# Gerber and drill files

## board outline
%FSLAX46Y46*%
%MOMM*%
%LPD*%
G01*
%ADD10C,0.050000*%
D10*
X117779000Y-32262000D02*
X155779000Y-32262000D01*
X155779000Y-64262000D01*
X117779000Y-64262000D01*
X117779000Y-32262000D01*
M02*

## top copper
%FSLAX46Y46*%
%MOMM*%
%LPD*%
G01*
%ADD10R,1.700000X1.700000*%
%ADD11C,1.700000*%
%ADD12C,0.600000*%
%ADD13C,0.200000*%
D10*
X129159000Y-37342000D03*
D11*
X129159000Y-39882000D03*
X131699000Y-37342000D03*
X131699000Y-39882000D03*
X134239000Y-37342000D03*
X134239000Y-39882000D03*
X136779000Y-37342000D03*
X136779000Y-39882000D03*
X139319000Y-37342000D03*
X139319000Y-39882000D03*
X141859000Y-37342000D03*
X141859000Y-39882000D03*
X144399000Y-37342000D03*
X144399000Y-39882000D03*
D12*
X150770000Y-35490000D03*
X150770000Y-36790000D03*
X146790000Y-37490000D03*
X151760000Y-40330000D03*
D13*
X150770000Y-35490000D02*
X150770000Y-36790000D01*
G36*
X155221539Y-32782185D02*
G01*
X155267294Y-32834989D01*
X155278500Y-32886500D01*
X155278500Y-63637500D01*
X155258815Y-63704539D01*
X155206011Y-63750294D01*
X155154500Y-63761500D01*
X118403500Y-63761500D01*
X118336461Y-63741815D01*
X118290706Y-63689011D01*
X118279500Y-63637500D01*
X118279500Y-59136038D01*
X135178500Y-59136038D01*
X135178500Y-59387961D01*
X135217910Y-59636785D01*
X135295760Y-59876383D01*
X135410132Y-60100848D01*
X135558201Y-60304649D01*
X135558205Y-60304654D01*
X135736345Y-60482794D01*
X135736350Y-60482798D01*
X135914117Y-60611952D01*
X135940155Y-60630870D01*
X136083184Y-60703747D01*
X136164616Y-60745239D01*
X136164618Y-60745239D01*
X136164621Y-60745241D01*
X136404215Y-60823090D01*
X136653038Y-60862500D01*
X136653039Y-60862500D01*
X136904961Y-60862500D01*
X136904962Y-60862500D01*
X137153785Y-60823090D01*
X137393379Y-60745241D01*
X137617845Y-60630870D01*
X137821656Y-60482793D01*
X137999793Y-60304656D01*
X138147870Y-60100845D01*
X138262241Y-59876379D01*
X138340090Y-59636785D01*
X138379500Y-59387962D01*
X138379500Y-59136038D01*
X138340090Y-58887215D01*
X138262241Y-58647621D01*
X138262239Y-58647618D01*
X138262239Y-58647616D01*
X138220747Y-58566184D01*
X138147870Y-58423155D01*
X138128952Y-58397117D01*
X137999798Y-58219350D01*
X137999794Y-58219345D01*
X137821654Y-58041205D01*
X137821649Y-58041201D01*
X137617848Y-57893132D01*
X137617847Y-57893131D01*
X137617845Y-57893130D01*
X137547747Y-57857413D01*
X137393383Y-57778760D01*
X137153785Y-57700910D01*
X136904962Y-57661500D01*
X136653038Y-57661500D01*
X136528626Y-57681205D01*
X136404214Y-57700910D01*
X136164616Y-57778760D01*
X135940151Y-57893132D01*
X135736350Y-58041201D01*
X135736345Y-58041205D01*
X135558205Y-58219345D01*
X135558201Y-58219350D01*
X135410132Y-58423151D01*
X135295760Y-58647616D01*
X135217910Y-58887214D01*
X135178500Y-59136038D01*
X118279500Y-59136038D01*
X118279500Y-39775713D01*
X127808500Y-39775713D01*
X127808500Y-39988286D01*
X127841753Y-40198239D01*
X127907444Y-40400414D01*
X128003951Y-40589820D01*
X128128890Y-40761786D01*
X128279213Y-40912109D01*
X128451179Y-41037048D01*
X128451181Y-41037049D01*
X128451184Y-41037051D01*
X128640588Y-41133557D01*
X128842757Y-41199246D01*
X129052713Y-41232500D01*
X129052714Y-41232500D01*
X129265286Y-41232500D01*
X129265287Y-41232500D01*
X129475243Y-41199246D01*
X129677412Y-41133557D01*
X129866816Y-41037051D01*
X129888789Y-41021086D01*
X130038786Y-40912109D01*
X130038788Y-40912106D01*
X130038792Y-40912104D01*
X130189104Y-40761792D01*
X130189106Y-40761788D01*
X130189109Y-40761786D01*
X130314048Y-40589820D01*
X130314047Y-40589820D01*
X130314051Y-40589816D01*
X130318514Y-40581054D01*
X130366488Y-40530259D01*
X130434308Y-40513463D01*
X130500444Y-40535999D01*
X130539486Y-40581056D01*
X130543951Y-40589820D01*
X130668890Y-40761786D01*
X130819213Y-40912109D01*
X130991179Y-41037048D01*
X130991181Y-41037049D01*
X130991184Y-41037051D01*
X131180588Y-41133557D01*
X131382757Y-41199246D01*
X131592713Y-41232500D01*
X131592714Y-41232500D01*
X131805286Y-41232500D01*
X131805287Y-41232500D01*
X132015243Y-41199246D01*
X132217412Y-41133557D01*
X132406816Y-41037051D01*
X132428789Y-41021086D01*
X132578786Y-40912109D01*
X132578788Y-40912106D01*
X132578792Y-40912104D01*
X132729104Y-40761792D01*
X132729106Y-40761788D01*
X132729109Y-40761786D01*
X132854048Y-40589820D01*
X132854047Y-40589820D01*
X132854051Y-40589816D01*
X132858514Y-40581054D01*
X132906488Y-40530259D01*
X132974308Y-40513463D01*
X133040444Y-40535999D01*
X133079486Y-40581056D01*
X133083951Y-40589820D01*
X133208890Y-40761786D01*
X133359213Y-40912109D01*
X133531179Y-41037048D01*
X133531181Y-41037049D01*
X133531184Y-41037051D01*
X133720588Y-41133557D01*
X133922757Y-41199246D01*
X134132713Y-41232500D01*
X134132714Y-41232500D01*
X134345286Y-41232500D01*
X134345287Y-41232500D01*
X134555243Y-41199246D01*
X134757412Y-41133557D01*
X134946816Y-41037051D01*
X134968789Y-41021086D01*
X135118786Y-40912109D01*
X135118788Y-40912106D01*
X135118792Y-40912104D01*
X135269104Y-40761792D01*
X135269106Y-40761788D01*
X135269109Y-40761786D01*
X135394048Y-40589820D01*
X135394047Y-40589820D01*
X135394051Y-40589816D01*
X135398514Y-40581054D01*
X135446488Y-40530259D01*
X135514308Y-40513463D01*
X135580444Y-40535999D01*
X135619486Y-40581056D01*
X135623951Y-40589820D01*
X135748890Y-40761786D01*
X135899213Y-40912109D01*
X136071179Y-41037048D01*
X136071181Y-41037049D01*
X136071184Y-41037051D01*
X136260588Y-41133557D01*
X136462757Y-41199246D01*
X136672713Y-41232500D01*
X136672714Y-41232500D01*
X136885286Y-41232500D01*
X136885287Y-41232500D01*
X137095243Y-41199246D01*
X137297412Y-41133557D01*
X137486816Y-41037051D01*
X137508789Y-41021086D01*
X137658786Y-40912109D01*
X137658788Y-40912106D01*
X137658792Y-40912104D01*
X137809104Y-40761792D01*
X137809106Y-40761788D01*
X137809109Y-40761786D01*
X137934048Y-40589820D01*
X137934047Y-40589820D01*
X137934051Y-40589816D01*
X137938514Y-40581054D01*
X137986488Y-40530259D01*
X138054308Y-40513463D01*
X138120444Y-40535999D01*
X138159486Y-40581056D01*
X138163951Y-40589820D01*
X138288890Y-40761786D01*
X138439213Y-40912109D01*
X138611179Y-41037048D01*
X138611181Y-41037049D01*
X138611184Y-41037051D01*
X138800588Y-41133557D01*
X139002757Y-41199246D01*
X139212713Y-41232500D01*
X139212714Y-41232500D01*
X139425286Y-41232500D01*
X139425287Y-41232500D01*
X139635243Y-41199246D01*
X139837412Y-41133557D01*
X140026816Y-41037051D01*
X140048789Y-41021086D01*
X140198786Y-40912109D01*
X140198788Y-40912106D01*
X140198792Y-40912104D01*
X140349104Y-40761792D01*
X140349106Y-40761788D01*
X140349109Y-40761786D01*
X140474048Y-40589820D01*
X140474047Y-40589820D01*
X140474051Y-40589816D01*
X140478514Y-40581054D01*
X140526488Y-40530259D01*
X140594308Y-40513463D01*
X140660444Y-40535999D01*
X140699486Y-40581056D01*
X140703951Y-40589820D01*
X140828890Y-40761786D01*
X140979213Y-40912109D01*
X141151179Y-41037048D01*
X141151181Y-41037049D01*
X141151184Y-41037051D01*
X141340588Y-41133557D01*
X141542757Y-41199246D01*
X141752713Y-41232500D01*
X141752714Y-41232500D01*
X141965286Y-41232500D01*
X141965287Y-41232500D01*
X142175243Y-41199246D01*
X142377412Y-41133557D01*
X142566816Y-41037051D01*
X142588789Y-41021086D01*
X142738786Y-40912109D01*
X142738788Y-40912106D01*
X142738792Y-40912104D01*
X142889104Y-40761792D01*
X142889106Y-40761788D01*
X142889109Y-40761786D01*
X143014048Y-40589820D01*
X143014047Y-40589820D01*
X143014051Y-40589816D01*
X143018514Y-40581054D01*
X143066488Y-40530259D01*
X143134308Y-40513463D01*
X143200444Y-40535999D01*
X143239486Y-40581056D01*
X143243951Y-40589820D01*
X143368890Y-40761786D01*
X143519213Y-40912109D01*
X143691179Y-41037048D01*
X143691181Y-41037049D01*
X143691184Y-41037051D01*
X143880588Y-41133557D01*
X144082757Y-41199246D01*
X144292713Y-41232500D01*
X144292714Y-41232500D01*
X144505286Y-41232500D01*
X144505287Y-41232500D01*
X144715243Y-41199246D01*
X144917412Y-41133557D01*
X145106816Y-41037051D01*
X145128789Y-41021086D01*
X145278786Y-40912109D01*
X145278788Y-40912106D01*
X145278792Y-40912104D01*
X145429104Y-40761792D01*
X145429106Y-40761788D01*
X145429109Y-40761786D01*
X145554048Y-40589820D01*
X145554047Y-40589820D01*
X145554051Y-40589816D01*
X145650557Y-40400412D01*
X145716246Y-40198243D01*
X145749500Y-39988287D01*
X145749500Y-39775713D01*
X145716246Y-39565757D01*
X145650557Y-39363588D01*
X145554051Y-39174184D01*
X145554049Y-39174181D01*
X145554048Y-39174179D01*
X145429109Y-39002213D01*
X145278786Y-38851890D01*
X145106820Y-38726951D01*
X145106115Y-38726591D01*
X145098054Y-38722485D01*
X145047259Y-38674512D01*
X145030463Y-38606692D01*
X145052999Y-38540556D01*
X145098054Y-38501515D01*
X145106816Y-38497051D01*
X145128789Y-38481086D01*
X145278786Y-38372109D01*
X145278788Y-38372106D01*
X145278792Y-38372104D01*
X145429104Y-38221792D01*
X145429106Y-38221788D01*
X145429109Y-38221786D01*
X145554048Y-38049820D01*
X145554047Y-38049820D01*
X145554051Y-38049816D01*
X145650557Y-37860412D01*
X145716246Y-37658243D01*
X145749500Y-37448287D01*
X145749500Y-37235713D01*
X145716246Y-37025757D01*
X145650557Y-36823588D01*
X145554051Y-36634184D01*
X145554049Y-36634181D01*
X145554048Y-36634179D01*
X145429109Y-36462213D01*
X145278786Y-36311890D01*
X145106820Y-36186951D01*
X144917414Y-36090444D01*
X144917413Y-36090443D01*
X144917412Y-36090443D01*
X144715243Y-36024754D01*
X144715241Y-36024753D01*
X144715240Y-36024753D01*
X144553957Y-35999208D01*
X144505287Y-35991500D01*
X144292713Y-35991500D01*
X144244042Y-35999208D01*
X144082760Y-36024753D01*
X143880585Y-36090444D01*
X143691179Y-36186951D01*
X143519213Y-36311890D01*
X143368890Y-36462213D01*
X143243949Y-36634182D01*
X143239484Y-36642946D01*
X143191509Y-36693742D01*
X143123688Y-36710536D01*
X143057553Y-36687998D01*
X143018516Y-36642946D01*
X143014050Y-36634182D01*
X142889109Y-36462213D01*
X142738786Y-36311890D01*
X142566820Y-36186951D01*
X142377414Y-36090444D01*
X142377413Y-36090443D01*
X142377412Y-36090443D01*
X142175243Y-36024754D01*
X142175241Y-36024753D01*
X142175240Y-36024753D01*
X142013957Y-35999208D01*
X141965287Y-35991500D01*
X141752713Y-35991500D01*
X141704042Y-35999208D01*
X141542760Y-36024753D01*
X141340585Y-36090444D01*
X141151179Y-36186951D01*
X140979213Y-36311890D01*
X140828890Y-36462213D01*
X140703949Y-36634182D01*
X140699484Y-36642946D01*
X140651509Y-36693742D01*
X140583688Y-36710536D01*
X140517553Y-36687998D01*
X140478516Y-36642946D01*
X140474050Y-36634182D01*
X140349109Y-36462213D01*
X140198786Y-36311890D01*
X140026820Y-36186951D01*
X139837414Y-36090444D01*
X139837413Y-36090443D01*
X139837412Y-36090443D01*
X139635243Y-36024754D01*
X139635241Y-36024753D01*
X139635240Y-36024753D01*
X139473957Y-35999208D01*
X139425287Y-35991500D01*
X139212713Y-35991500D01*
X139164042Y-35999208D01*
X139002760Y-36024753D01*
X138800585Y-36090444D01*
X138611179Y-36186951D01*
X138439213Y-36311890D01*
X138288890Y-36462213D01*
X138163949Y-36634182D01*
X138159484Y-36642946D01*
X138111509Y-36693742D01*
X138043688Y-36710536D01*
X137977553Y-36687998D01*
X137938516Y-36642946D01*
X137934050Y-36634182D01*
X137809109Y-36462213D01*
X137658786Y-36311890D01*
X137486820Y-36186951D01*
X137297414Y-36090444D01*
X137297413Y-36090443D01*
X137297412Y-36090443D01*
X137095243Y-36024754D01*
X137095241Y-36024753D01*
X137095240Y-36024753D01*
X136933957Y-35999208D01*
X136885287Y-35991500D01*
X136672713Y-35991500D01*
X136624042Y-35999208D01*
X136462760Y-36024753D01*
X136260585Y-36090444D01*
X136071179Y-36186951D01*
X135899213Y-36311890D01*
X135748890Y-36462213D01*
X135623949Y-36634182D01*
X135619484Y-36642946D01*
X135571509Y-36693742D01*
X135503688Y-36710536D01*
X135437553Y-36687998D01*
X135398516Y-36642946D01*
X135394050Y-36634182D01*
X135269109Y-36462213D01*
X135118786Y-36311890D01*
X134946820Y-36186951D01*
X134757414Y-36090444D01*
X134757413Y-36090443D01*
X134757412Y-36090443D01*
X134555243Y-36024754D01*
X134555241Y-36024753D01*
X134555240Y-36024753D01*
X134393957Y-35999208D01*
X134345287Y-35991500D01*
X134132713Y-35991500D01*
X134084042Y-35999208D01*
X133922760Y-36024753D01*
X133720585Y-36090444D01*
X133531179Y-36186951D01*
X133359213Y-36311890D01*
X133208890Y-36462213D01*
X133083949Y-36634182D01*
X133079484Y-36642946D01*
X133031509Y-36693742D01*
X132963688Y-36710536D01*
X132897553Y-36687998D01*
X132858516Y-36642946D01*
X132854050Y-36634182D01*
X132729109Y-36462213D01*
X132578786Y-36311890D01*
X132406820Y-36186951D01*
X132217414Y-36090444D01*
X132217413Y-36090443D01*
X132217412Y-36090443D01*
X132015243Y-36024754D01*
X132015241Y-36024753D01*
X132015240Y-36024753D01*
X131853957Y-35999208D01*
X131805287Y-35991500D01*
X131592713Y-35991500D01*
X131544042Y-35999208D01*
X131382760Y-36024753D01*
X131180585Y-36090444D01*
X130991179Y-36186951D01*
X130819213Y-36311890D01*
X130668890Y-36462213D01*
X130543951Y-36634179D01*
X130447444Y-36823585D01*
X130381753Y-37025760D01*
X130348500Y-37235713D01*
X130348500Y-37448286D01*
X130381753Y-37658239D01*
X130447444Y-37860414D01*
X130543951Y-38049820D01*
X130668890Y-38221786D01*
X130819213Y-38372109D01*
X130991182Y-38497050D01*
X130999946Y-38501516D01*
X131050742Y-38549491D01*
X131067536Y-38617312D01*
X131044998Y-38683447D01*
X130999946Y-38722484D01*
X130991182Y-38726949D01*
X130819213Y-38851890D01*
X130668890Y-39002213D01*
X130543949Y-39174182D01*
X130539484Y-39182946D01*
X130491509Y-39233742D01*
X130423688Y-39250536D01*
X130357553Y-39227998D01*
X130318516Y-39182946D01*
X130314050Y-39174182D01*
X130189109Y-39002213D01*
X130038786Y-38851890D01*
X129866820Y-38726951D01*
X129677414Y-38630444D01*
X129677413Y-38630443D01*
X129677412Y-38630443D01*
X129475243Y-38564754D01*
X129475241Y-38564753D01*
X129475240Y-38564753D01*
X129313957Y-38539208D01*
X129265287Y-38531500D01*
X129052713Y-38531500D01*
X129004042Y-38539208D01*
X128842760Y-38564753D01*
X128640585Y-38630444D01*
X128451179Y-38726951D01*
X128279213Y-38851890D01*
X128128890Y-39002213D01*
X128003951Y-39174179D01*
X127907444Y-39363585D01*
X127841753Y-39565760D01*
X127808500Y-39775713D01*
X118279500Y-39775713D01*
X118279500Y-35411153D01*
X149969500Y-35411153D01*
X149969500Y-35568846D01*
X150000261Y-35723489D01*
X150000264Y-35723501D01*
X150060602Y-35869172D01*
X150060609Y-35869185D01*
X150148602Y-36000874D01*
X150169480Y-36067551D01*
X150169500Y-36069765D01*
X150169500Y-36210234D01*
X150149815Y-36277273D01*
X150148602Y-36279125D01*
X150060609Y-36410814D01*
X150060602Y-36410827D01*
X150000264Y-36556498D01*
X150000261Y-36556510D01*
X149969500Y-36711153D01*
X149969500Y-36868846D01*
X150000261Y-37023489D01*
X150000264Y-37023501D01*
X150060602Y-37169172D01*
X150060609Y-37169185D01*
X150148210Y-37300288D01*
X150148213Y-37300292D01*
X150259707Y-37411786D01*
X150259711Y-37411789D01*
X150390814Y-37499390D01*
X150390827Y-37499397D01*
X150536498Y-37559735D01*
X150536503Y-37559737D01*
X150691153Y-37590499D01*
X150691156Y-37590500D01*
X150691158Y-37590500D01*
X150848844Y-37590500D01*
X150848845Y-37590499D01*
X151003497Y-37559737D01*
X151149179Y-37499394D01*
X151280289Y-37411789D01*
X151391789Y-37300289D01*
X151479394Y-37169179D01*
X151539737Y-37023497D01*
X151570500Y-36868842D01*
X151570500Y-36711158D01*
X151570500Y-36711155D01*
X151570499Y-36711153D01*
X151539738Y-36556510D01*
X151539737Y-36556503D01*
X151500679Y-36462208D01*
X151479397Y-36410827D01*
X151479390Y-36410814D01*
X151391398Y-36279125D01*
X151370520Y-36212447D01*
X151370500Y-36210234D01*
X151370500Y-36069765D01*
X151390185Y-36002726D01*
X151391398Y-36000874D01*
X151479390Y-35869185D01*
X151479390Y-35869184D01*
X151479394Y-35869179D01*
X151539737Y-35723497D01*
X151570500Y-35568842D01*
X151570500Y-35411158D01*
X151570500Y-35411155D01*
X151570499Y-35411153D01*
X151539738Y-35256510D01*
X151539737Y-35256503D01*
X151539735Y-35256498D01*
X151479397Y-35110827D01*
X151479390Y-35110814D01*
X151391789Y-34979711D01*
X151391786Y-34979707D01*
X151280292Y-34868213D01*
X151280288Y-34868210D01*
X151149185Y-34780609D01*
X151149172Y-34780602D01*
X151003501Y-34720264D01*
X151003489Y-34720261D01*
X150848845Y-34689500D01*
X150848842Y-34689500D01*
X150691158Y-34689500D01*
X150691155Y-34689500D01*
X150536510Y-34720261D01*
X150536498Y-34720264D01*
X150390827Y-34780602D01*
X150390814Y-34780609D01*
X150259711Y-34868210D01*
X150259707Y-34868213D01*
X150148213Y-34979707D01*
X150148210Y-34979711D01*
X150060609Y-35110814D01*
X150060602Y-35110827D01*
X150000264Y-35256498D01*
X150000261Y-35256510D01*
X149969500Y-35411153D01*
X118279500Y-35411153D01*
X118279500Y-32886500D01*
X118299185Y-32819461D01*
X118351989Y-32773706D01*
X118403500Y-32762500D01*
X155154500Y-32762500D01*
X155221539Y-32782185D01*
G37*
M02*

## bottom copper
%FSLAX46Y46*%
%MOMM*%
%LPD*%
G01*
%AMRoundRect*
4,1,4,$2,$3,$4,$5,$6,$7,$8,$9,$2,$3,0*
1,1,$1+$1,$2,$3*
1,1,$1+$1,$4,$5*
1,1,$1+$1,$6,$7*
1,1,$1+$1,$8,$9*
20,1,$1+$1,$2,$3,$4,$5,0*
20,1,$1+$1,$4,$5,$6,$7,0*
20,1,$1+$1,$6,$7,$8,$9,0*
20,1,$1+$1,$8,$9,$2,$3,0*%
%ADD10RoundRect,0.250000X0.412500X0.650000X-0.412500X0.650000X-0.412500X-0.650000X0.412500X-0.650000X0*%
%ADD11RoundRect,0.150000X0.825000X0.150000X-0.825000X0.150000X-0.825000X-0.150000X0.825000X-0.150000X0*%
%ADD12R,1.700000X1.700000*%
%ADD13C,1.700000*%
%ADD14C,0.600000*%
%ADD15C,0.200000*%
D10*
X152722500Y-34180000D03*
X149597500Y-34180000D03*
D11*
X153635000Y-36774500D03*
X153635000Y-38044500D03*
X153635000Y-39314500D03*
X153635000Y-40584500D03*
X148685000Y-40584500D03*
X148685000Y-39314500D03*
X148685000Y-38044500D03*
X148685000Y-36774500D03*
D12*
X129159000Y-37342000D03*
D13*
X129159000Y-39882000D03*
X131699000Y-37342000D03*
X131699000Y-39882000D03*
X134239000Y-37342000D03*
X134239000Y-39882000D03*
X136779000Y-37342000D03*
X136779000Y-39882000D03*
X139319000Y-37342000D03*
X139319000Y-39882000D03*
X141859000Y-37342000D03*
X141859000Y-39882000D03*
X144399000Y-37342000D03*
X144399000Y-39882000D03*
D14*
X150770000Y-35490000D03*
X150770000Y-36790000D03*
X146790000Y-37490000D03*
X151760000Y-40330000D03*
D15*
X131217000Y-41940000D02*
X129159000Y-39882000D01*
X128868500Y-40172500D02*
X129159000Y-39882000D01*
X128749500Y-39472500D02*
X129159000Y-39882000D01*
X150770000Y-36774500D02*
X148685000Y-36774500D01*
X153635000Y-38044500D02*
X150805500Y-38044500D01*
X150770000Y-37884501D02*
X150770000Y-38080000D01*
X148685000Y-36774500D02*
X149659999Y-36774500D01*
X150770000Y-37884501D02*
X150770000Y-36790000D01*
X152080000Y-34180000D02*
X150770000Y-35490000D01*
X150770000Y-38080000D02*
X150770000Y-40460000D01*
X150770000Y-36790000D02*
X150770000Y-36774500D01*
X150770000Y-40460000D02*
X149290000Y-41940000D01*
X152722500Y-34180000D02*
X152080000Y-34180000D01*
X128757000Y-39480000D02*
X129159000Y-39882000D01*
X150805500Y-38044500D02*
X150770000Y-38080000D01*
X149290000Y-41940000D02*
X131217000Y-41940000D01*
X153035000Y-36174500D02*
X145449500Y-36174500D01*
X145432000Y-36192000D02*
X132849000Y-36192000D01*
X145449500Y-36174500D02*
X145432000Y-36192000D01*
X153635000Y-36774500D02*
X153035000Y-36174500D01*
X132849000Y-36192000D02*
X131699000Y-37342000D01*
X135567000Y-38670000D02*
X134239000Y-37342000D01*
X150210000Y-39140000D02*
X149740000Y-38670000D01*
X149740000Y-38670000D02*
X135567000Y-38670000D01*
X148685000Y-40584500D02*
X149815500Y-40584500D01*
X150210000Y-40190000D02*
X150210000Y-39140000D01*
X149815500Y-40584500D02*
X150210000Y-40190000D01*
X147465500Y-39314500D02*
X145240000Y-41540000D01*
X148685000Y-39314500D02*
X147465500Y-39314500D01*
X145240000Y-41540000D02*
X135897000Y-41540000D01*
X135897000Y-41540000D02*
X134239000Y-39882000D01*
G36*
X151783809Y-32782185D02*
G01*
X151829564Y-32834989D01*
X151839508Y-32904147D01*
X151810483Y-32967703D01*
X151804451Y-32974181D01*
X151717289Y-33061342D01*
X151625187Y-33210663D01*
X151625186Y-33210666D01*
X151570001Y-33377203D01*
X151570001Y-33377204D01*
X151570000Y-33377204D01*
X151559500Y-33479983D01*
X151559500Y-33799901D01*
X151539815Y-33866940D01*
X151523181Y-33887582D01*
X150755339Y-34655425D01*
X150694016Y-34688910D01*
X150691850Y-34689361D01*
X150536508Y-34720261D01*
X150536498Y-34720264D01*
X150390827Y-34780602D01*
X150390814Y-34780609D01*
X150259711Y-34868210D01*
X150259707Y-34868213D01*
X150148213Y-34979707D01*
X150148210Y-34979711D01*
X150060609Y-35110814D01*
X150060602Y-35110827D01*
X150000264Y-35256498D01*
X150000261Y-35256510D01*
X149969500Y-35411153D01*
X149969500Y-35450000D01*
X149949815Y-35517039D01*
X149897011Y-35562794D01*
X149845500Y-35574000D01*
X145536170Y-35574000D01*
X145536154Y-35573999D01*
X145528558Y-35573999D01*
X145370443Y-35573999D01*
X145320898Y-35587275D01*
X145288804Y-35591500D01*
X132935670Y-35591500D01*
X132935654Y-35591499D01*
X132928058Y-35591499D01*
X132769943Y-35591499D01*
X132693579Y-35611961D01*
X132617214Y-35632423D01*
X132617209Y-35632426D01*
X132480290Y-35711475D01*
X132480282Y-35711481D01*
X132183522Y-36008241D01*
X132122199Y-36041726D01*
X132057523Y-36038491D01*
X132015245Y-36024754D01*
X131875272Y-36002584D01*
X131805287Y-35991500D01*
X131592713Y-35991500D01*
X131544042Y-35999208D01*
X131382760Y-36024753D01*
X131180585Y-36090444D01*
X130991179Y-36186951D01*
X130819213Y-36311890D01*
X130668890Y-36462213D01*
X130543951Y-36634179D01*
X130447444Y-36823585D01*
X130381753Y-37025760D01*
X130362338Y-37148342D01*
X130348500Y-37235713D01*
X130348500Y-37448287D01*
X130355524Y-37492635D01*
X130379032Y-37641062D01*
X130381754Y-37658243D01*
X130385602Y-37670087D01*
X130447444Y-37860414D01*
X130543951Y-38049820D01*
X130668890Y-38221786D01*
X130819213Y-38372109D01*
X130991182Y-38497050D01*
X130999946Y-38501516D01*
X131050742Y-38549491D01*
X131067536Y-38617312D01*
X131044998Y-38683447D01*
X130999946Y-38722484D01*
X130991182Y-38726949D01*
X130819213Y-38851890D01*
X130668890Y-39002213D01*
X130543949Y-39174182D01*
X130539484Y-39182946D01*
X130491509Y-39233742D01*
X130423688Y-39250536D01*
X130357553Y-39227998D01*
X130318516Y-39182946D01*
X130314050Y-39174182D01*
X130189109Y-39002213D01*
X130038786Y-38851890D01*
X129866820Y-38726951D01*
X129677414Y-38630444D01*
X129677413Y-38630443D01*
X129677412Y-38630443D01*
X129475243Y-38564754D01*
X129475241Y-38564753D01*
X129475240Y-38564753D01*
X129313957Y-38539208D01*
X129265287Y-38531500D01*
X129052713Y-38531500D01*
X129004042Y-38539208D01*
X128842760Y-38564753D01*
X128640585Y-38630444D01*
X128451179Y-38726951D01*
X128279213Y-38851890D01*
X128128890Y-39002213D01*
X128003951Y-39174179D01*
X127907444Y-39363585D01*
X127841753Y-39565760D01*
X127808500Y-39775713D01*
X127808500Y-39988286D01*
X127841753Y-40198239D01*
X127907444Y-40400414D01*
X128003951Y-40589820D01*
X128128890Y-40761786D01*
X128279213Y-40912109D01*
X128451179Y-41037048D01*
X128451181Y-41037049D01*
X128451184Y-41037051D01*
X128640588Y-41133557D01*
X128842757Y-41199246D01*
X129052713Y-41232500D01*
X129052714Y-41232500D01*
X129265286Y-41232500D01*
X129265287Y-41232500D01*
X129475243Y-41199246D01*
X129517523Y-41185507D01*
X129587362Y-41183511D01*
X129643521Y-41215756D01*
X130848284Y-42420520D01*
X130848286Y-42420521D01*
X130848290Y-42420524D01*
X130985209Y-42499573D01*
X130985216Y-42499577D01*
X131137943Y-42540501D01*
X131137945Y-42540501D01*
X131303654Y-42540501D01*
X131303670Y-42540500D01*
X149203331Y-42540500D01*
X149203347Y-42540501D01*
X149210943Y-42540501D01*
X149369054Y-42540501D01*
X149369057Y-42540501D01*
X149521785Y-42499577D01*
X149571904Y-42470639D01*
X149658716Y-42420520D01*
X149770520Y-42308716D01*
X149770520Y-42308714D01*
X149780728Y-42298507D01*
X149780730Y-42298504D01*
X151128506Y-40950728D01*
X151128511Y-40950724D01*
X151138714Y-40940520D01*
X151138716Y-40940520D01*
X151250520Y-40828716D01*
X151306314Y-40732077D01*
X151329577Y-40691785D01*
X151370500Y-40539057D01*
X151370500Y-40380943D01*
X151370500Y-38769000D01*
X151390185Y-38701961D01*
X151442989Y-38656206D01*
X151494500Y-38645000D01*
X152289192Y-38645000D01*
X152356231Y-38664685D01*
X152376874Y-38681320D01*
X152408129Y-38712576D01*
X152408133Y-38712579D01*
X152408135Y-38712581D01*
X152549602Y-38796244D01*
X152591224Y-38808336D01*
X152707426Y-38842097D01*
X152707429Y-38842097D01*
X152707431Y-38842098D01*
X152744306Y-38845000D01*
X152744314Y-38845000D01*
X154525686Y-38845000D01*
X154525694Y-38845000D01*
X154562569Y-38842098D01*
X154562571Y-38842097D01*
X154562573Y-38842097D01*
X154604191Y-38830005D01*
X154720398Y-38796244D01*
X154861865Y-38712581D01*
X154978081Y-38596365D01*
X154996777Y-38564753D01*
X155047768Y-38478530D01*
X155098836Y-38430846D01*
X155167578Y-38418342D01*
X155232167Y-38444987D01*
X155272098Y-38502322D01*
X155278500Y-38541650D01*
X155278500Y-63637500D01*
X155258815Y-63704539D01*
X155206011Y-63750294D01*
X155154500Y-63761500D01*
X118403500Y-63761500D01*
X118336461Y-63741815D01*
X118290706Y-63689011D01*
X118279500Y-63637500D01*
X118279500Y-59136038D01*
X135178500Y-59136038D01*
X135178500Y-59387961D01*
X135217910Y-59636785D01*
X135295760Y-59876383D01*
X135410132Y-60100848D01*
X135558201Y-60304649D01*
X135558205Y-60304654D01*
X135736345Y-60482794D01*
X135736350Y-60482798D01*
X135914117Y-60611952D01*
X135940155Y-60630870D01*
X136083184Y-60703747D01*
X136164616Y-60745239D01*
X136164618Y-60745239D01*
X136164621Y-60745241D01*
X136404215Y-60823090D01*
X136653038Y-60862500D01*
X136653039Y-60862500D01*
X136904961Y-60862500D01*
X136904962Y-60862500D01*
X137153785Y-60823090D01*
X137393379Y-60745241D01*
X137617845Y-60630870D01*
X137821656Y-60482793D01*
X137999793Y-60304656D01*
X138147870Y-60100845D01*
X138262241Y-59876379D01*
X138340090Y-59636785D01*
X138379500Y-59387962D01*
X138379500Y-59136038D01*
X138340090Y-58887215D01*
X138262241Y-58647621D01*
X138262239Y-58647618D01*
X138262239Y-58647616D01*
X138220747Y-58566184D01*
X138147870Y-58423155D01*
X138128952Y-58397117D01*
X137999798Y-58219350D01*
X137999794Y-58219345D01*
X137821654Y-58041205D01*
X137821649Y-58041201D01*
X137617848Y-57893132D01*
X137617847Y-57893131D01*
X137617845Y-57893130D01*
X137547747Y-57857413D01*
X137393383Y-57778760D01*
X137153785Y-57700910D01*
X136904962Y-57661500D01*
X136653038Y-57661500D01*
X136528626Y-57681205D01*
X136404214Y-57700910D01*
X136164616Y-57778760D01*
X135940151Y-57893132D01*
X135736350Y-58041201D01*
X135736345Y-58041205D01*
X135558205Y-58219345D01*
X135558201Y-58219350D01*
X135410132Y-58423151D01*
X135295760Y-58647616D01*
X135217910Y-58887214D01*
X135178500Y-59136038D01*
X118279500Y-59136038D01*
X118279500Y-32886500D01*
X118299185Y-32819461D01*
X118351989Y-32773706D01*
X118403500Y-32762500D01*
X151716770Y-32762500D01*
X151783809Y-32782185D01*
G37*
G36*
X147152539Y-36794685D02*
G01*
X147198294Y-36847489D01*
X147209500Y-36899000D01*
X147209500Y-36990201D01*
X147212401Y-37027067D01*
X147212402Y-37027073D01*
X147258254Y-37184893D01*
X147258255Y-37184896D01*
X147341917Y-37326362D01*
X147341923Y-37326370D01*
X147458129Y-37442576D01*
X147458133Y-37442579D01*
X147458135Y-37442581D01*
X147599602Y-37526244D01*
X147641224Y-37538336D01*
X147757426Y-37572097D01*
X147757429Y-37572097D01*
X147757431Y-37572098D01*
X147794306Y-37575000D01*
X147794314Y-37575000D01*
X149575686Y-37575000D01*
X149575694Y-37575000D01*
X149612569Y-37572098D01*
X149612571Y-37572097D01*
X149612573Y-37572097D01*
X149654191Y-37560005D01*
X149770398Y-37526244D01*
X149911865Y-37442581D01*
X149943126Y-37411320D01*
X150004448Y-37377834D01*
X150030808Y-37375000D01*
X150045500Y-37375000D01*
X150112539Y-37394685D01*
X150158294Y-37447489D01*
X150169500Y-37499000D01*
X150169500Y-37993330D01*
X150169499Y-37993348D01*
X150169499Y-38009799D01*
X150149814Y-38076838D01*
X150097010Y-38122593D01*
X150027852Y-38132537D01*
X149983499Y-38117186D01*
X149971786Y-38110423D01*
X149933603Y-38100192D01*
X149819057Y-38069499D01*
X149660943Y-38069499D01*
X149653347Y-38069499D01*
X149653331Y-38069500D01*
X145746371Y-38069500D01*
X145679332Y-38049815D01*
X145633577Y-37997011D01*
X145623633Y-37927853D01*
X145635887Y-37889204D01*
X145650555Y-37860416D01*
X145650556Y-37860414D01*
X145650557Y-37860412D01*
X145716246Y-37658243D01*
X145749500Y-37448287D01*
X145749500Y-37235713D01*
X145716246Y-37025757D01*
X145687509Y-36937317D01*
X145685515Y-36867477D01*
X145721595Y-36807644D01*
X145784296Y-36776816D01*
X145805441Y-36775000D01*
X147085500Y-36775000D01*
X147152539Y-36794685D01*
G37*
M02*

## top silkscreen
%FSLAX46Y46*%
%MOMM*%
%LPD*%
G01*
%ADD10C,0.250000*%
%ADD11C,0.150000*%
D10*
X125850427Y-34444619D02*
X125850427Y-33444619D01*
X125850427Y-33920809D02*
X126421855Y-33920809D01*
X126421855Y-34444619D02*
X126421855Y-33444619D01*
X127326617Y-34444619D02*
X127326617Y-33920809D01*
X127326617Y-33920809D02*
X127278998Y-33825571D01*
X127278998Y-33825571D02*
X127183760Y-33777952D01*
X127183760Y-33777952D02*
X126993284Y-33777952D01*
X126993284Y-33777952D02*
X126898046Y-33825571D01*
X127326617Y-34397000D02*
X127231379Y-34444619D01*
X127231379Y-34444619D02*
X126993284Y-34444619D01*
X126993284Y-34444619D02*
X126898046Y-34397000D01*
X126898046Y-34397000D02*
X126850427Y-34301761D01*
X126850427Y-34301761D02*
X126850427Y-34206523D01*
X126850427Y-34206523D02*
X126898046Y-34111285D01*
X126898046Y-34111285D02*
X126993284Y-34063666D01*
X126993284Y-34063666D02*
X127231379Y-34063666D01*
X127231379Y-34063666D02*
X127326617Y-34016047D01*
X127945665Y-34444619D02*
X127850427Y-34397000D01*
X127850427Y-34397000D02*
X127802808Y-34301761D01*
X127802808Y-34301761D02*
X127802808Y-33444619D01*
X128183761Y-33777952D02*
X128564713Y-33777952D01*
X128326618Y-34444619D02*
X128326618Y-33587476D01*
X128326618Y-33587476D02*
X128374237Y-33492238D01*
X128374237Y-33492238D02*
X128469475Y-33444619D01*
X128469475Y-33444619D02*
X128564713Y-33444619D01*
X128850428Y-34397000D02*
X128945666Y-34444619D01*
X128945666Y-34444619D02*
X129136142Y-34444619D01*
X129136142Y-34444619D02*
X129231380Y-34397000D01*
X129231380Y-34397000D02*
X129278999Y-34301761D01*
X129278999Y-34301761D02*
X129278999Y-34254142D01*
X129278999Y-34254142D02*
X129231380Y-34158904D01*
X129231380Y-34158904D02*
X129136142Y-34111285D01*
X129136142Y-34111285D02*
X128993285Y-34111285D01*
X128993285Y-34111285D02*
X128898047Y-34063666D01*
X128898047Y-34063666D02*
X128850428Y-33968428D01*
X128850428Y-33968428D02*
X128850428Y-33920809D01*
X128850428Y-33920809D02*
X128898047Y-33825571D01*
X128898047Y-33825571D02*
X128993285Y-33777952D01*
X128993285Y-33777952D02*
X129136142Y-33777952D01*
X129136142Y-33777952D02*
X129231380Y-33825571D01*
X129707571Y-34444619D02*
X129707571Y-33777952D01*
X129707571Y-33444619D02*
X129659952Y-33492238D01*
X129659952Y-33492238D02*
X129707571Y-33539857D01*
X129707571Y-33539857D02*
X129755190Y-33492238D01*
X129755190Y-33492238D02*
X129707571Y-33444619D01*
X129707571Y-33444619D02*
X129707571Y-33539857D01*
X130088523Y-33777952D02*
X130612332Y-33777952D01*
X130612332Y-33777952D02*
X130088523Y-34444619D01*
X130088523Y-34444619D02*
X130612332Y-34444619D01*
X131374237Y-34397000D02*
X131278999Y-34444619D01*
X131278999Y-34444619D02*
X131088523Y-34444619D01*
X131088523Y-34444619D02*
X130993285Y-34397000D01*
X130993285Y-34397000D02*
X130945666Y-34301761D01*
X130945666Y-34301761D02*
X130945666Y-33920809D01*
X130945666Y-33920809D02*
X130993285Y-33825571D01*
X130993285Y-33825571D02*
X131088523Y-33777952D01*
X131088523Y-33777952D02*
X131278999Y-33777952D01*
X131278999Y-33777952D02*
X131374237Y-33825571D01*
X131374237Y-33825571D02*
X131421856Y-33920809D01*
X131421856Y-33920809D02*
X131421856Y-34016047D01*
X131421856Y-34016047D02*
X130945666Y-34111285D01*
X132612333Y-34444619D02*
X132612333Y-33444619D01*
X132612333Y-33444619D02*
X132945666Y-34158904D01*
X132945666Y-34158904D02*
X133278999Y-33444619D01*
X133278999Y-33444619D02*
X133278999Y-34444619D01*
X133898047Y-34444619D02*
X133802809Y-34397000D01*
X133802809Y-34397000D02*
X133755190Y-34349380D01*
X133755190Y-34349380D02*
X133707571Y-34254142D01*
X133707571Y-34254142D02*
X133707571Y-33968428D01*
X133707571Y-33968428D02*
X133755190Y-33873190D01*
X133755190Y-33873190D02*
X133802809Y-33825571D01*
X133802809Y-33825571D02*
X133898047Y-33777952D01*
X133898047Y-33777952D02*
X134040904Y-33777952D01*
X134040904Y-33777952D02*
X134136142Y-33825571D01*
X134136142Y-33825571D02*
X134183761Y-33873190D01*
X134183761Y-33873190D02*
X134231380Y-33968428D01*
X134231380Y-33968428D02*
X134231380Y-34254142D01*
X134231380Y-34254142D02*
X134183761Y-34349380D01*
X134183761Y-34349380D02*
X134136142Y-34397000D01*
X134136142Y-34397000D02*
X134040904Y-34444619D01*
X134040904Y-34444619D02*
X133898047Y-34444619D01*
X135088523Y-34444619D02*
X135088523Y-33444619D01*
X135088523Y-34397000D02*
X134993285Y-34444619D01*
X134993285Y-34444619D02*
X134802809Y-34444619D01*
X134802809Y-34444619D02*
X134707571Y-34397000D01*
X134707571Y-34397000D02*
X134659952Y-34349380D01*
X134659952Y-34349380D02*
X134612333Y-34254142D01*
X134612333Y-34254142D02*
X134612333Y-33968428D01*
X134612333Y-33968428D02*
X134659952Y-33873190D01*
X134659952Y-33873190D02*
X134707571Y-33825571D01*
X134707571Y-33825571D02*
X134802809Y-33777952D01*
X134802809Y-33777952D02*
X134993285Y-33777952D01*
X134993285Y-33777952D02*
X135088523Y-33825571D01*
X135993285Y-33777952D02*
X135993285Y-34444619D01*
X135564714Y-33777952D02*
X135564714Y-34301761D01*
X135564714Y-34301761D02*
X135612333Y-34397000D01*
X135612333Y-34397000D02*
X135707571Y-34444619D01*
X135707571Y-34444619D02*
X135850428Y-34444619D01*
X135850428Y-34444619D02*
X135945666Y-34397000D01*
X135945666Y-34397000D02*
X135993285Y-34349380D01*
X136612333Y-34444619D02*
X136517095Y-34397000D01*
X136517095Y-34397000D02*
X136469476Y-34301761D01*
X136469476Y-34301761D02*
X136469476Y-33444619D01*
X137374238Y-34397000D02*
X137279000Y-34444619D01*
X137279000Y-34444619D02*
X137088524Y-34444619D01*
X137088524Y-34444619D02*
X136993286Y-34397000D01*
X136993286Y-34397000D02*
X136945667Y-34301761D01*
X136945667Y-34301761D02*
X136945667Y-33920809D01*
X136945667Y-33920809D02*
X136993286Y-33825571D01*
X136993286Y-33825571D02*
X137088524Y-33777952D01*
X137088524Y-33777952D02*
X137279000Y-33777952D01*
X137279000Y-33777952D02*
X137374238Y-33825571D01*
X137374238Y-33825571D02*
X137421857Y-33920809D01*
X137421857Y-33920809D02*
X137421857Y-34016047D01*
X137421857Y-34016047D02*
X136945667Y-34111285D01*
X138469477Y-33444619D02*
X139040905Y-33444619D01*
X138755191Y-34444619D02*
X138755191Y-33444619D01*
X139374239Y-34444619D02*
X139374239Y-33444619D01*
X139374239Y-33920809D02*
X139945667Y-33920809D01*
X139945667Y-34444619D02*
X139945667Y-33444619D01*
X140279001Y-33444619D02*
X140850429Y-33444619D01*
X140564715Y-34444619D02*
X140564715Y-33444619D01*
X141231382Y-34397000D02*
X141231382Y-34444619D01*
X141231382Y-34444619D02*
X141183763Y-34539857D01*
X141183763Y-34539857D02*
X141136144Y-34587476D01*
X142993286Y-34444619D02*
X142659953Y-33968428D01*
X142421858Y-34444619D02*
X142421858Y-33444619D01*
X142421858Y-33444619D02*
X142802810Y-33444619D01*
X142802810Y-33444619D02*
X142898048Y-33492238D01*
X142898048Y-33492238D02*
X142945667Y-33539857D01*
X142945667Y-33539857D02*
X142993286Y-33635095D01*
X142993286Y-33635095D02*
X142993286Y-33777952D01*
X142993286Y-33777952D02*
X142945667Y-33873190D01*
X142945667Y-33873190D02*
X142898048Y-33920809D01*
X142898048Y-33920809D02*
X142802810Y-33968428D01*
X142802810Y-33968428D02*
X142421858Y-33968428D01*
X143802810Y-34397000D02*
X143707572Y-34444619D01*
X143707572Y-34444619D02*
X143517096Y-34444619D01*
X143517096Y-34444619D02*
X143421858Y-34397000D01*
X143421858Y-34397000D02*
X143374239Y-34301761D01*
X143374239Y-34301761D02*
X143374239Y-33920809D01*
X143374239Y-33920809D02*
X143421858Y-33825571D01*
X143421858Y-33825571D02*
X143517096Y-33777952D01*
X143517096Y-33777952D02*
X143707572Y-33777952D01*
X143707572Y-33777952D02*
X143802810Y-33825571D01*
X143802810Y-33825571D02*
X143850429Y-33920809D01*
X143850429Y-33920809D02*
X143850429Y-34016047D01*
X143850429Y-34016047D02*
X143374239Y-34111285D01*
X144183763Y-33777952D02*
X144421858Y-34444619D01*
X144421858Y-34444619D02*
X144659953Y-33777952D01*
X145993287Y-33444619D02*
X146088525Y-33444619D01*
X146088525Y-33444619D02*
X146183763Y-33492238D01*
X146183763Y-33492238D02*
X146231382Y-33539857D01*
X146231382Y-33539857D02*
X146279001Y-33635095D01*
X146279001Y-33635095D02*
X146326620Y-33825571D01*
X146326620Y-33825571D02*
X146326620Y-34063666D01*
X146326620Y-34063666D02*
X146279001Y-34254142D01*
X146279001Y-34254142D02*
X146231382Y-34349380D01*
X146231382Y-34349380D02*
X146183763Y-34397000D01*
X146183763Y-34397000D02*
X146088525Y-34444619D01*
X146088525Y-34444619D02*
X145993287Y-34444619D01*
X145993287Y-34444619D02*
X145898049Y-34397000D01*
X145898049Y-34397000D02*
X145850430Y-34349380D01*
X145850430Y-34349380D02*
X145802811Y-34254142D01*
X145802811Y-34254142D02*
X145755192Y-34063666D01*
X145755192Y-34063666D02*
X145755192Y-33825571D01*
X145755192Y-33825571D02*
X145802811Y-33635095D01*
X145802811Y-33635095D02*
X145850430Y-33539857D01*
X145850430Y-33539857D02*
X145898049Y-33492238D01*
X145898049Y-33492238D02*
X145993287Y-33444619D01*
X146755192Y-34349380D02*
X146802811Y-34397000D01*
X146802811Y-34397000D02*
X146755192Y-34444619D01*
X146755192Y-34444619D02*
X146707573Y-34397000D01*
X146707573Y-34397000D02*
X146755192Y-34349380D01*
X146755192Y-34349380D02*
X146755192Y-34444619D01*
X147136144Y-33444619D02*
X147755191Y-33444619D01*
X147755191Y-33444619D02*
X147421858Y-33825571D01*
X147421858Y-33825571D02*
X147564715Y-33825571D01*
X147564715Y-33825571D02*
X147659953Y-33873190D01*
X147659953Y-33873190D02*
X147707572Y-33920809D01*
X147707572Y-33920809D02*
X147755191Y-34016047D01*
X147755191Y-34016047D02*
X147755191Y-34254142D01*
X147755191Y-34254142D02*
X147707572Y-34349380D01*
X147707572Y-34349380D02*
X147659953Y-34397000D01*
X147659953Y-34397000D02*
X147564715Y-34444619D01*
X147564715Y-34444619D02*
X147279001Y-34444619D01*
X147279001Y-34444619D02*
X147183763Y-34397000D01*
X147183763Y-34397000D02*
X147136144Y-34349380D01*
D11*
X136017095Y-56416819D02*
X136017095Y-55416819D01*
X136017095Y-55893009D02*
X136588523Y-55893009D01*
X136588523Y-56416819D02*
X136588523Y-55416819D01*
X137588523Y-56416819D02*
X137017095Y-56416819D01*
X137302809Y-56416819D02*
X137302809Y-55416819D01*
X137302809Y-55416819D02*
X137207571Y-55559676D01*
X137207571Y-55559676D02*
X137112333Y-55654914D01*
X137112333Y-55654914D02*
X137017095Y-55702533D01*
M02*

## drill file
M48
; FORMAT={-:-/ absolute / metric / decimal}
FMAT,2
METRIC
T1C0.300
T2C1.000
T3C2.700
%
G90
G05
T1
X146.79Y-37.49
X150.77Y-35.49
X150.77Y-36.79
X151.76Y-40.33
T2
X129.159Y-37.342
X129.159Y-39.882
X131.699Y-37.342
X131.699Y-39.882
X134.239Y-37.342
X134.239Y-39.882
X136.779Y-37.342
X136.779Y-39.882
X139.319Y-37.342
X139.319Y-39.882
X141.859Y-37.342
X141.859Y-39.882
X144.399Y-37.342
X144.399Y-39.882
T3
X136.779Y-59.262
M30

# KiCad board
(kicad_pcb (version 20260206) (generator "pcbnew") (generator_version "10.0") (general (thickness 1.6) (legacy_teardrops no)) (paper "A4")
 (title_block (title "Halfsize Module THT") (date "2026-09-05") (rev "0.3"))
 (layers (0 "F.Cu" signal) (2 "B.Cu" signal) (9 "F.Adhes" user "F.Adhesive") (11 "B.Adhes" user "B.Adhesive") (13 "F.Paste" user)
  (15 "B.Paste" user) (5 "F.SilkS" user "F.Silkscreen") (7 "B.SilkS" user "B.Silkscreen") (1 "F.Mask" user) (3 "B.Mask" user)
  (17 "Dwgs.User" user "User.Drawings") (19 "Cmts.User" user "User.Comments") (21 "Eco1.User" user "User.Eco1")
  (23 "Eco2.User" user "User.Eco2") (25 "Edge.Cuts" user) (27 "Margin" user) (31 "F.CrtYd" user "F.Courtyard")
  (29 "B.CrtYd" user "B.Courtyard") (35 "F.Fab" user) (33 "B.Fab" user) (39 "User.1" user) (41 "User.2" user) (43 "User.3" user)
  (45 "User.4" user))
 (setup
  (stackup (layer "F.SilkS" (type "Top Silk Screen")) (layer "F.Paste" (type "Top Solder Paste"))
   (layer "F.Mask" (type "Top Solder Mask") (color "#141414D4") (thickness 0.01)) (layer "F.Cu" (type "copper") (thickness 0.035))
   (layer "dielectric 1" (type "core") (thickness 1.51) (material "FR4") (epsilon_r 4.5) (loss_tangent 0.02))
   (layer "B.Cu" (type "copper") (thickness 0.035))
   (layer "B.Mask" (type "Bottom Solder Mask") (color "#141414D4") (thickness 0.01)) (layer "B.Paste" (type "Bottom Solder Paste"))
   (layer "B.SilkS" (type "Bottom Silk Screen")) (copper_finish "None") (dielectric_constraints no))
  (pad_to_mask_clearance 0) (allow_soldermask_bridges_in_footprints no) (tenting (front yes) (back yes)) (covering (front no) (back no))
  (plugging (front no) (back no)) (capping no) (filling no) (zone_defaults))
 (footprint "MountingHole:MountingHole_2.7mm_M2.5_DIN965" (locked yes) (layer "F.Cu") (at 136.779 59.262)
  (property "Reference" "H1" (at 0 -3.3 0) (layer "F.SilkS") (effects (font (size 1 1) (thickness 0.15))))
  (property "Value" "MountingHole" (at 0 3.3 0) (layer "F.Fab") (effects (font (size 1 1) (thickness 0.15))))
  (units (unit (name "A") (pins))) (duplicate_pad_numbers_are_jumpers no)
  (pad "" np_thru_hole circle (at 0 0) (size 2.7 2.7) (drill 2.7) (layers "*.Cu" "*.Mask")))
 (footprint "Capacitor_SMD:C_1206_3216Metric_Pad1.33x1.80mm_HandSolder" (layer "B.Cu") (at 151.16 34.18 180)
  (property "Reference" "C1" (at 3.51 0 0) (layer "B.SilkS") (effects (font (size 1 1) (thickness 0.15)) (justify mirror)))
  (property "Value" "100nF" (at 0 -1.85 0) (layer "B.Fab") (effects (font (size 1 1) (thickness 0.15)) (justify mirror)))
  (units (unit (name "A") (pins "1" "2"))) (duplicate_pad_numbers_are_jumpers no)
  (pad "1" smd roundrect (at -1.5625 0 180) (size 1.325 1.8) (layers "B.Cu" "B.Mask" "B.Paste") (roundrect_rratio 0.188679) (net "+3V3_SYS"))
  (pad "2" smd roundrect (at 1.5625 0 180) (size 1.325 1.8) (layers "B.Cu" "B.Mask" "B.Paste") (roundrect_rratio 0.188679) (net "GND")
   (zone_connect 2)))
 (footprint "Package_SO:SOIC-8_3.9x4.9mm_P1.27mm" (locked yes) (layer "B.Cu") (at 151.16 38.6795 180)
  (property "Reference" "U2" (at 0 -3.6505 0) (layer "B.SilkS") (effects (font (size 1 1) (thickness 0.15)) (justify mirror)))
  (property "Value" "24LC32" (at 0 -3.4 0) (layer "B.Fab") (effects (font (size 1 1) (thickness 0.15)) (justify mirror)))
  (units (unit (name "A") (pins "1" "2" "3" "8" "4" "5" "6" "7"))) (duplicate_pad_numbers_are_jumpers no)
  (pad "1" smd roundrect (at -2.475 1.905 180) (size 1.95 0.6) (layers "B.Cu" "B.Mask" "B.Paste") (roundrect_rratio 0.25) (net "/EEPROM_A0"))
  (pad "2" smd roundrect (at -2.475 0.635 180) (size 1.95 0.6) (layers "B.Cu" "B.Mask" "B.Paste") (roundrect_rratio 0.25) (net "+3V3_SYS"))
  (pad "3" smd roundrect (at -2.475 -0.635 180) (size 1.95 0.6) (layers "B.Cu" "B.Mask" "B.Paste") (roundrect_rratio 0.25) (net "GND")
   (zone_connect 2))
  (pad "4" smd roundrect (at -2.475 -1.905 180) (size 1.95 0.6) (layers "B.Cu" "B.Mask" "B.Paste") (roundrect_rratio 0.25) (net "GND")
   (zone_connect 2))
  (pad "5" smd roundrect (at 2.475 -1.905 180) (size 1.95 0.6) (layers "B.Cu" "B.Mask" "B.Paste") (roundrect_rratio 0.25) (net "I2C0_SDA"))
  (pad "6" smd roundrect (at 2.475 -0.635 180) (size 1.95 0.6) (layers "B.Cu" "B.Mask" "B.Paste") (roundrect_rratio 0.25) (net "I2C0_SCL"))
  (pad "7" smd roundrect (at 2.475 0.635 180) (size 1.95 0.6) (layers "B.Cu" "B.Mask" "B.Paste") (roundrect_rratio 0.25) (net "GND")
   (zone_connect 2))
  (pad "8" smd roundrect (at 2.475 1.905 180) (size 1.95 0.6) (layers "B.Cu" "B.Mask" "B.Paste") (roundrect_rratio 0.25) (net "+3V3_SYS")))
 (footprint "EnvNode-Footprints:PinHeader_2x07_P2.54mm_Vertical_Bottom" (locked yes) (layer "B.Cu") (at 129.159 37.342 -90)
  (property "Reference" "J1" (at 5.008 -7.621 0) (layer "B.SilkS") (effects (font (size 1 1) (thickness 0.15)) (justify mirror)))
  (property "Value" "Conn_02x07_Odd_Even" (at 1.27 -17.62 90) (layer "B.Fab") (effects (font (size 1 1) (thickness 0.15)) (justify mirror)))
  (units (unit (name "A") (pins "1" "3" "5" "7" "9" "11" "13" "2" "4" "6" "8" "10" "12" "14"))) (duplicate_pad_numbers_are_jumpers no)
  (pad "1" thru_hole rect (at 0 0 270) (size 1.7 1.7) (drill 1) (layers "*.Cu" "*.Mask") (remove_unused_layers no) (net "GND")
   (zone_connect 2))
  (pad "2" thru_hole circle (at 2.54 0 270) (size 1.7 1.7) (drill 1) (layers "*.Cu" "*.Mask") (remove_unused_layers no) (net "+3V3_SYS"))
  (pad "3" thru_hole circle (at 0 -2.54 270) (size 1.7 1.7) (drill 1) (layers "*.Cu" "*.Mask") (remove_unused_layers no) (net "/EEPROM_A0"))
  (pad "4" thru_hole circle (at 2.54 -2.54 270) (size 1.7 1.7) (drill 1) (layers "*.Cu" "*.Mask") (remove_unused_layers no) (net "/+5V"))
  (pad "5" thru_hole circle (at 0 -5.08 270) (size 1.7 1.7) (drill 1) (layers "*.Cu" "*.Mask") (remove_unused_layers no) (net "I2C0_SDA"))
  (pad "6" thru_hole circle (at 2.54 -5.08 270) (size 1.7 1.7) (drill 1) (layers "*.Cu" "*.Mask") (remove_unused_layers no) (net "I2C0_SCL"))
  (pad "7" thru_hole circle (at 0 -7.62 270) (size 1.7 1.7) (drill 1) (layers "*.Cu" "*.Mask") (remove_unused_layers no) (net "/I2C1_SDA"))
  (pad "8" thru_hole circle (at 2.54 -7.62 270) (size 1.7 1.7) (drill 1) (layers "*.Cu" "*.Mask") (remove_unused_layers no)
   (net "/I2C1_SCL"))
  (pad "9" thru_hole circle (at 0 -10.16 270) (size 1.7 1.7) (drill 1) (layers "*.Cu" "*.Mask") (remove_unused_layers no) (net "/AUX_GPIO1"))
  (pad "10" thru_hole circle (at 2.54 -10.16 270) (size 1.7 1.7) (drill 1) (layers "*.Cu" "*.Mask") (remove_unused_layers no)
   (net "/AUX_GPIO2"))
  (pad "11" thru_hole circle (at 0 -12.7 270) (size 1.7 1.7) (drill 1) (layers "*.Cu" "*.Mask") (remove_unused_layers no) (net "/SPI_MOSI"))
  (pad "12" thru_hole circle (at 2.54 -12.7 270) (size 1.7 1.7) (drill 1) (layers "*.Cu" "*.Mask") (remove_unused_layers no)
   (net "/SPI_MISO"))
  (pad "13" thru_hole circle (at 0 -15.24 270) (size 1.7 1.7) (drill 1) (layers "*.Cu" "*.Mask") (remove_unused_layers no) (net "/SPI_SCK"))
  (pad "14" thru_hole circle (at 2.54 -15.24 270) (size 1.7 1.7) (drill 1) (layers "*.Cu" "*.Mask") (remove_unused_layers no)
   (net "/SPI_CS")))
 (gr_rect (start 117.779 32.262) (end 155.779 64.262) (stroke (width 0.05) (type solid)) (fill no) (locked yes) (layer "Edge.Cuts"))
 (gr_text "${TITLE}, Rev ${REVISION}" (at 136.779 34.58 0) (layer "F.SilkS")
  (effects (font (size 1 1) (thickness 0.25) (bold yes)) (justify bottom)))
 (segment (start 150.77 35.49) (end 150.77 36.79) (width 0.2) (layer "F.Cu") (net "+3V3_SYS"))
 (via (at 150.77 35.49) (size 0.6) (drill 0.3) (layers "F.Cu" "B.Cu") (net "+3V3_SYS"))
 (via (at 150.77 36.79) (size 0.6) (drill 0.3) (layers "F.Cu" "B.Cu") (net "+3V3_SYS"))
 (segment (start 131.217 41.94) (end 129.159 39.882) (width 0.2) (layer "B.Cu") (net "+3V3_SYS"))
 (segment (start 128.8685 40.1725) (end 129.159 39.882) (width 0.2) (layer "B.Cu") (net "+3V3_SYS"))
 (segment (start 128.7495 39.4725) (end 129.159 39.882) (width 0.2) (layer "B.Cu") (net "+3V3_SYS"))
 (segment (start 150.77 36.7745) (end 148.685 36.7745) (width 0.2) (layer "B.Cu") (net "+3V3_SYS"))
 (segment (start 153.635 38.0445) (end 150.8055 38.0445) (width 0.2) (layer "B.Cu") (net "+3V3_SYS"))
 (segment (start 150.77 37.884501) (end 150.77 38.08) (width 0.2) (layer "B.Cu") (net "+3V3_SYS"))
 (segment (start 148.685 36.7745) (end 149.659999 36.7745) (width 0.2) (layer "B.Cu") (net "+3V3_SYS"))
 (segment (start 150.77 37.884501) (end 150.77 36.79) (width 0.2) (layer "B.Cu") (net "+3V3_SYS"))
 (segment (start 152.08 34.18) (end 150.77 35.49) (width 0.2) (layer "B.Cu") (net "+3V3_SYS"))
 (segment (start 150.77 38.08) (end 150.77 40.46) (width 0.2) (layer "B.Cu") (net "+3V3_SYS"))
 (segment (start 150.77 36.79) (end 150.77 36.7745) (width 0.2) (layer "B.Cu") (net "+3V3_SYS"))
 (segment (start 150.77 40.46) (end 149.29 41.94) (width 0.2) (layer "B.Cu") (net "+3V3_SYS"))
 (segment (start 152.7225 34.18) (end 152.08 34.18) (width 0.2) (layer "B.Cu") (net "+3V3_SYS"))
 (segment (start 128.757 39.48) (end 129.159 39.882) (width 0.2) (layer "B.Cu") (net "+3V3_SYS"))
 (segment (start 150.8055 38.0445) (end 150.77 38.08) (width 0.2) (layer "B.Cu") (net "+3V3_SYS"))
 (segment (start 149.29 41.94) (end 131.217 41.94) (width 0.2) (layer "B.Cu") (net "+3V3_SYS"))
 (via (at 146.79 37.49) (size 0.6) (drill 0.3) (layers "F.Cu" "B.Cu") (free yes) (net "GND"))
 (via (at 151.76 40.33) (size 0.6) (drill 0.3) (layers "F.Cu" "B.Cu") (free yes) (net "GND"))
 (segment (start 153.035 36.1745) (end 145.4495 36.1745) (width 0.2) (layer "B.Cu") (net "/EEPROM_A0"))
 (segment (start 145.432 36.192) (end 132.849 36.192) (width 0.2) (layer "B.Cu") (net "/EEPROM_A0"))
 (segment (start 145.4495 36.1745) (end 145.432 36.192) (width 0.2) (layer "B.Cu") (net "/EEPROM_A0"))
 (segment (start 153.635 36.7745) (end 153.035 36.1745) (width 0.2) (layer "B.Cu") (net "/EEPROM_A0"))
 (segment (start 132.849 36.192) (end 131.699 37.342) (width 0.2) (layer "B.Cu") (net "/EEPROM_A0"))
 (segment (start 135.567 38.67) (end 134.239 37.342) (width 0.2) (layer "B.Cu") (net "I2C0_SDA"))
 (segment (start 150.21 39.14) (end 149.74 38.67) (width 0.2) (layer "B.Cu") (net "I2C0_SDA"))
 (segment (start 149.74 38.67) (end 135.567 38.67) (width 0.2) (layer "B.Cu") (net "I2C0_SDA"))
 (segment (start 148.685 40.5845) (end 149.8155 40.5845) (width 0.2) (layer "B.Cu") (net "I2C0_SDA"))
 (segment (start 150.21 40.19) (end 150.21 39.14) (width 0.2) (layer "B.Cu") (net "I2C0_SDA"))
 (segment (start 149.8155 40.5845) (end 150.21 40.19) (width 0.2) (layer "B.Cu") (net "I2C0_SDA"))
 (segment (start 147.4655 39.3145) (end 145.24 41.54) (width 0.2) (layer "B.Cu") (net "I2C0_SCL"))
 (segment (start 148.685 39.3145) (end 147.4655 39.3145) (width 0.2) (layer "B.Cu") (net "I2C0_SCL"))
 (segment (start 145.24 41.54) (end 135.897 41.54) (width 0.2) (layer "B.Cu") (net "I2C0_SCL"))
 (segment (start 135.897 41.54) (end 134.239 39.882) (width 0.2) (layer "B.Cu") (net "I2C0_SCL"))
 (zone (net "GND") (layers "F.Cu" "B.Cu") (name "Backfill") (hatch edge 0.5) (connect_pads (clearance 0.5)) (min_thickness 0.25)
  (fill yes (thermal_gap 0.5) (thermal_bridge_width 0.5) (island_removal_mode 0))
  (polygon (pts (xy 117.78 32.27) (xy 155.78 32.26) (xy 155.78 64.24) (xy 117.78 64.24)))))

